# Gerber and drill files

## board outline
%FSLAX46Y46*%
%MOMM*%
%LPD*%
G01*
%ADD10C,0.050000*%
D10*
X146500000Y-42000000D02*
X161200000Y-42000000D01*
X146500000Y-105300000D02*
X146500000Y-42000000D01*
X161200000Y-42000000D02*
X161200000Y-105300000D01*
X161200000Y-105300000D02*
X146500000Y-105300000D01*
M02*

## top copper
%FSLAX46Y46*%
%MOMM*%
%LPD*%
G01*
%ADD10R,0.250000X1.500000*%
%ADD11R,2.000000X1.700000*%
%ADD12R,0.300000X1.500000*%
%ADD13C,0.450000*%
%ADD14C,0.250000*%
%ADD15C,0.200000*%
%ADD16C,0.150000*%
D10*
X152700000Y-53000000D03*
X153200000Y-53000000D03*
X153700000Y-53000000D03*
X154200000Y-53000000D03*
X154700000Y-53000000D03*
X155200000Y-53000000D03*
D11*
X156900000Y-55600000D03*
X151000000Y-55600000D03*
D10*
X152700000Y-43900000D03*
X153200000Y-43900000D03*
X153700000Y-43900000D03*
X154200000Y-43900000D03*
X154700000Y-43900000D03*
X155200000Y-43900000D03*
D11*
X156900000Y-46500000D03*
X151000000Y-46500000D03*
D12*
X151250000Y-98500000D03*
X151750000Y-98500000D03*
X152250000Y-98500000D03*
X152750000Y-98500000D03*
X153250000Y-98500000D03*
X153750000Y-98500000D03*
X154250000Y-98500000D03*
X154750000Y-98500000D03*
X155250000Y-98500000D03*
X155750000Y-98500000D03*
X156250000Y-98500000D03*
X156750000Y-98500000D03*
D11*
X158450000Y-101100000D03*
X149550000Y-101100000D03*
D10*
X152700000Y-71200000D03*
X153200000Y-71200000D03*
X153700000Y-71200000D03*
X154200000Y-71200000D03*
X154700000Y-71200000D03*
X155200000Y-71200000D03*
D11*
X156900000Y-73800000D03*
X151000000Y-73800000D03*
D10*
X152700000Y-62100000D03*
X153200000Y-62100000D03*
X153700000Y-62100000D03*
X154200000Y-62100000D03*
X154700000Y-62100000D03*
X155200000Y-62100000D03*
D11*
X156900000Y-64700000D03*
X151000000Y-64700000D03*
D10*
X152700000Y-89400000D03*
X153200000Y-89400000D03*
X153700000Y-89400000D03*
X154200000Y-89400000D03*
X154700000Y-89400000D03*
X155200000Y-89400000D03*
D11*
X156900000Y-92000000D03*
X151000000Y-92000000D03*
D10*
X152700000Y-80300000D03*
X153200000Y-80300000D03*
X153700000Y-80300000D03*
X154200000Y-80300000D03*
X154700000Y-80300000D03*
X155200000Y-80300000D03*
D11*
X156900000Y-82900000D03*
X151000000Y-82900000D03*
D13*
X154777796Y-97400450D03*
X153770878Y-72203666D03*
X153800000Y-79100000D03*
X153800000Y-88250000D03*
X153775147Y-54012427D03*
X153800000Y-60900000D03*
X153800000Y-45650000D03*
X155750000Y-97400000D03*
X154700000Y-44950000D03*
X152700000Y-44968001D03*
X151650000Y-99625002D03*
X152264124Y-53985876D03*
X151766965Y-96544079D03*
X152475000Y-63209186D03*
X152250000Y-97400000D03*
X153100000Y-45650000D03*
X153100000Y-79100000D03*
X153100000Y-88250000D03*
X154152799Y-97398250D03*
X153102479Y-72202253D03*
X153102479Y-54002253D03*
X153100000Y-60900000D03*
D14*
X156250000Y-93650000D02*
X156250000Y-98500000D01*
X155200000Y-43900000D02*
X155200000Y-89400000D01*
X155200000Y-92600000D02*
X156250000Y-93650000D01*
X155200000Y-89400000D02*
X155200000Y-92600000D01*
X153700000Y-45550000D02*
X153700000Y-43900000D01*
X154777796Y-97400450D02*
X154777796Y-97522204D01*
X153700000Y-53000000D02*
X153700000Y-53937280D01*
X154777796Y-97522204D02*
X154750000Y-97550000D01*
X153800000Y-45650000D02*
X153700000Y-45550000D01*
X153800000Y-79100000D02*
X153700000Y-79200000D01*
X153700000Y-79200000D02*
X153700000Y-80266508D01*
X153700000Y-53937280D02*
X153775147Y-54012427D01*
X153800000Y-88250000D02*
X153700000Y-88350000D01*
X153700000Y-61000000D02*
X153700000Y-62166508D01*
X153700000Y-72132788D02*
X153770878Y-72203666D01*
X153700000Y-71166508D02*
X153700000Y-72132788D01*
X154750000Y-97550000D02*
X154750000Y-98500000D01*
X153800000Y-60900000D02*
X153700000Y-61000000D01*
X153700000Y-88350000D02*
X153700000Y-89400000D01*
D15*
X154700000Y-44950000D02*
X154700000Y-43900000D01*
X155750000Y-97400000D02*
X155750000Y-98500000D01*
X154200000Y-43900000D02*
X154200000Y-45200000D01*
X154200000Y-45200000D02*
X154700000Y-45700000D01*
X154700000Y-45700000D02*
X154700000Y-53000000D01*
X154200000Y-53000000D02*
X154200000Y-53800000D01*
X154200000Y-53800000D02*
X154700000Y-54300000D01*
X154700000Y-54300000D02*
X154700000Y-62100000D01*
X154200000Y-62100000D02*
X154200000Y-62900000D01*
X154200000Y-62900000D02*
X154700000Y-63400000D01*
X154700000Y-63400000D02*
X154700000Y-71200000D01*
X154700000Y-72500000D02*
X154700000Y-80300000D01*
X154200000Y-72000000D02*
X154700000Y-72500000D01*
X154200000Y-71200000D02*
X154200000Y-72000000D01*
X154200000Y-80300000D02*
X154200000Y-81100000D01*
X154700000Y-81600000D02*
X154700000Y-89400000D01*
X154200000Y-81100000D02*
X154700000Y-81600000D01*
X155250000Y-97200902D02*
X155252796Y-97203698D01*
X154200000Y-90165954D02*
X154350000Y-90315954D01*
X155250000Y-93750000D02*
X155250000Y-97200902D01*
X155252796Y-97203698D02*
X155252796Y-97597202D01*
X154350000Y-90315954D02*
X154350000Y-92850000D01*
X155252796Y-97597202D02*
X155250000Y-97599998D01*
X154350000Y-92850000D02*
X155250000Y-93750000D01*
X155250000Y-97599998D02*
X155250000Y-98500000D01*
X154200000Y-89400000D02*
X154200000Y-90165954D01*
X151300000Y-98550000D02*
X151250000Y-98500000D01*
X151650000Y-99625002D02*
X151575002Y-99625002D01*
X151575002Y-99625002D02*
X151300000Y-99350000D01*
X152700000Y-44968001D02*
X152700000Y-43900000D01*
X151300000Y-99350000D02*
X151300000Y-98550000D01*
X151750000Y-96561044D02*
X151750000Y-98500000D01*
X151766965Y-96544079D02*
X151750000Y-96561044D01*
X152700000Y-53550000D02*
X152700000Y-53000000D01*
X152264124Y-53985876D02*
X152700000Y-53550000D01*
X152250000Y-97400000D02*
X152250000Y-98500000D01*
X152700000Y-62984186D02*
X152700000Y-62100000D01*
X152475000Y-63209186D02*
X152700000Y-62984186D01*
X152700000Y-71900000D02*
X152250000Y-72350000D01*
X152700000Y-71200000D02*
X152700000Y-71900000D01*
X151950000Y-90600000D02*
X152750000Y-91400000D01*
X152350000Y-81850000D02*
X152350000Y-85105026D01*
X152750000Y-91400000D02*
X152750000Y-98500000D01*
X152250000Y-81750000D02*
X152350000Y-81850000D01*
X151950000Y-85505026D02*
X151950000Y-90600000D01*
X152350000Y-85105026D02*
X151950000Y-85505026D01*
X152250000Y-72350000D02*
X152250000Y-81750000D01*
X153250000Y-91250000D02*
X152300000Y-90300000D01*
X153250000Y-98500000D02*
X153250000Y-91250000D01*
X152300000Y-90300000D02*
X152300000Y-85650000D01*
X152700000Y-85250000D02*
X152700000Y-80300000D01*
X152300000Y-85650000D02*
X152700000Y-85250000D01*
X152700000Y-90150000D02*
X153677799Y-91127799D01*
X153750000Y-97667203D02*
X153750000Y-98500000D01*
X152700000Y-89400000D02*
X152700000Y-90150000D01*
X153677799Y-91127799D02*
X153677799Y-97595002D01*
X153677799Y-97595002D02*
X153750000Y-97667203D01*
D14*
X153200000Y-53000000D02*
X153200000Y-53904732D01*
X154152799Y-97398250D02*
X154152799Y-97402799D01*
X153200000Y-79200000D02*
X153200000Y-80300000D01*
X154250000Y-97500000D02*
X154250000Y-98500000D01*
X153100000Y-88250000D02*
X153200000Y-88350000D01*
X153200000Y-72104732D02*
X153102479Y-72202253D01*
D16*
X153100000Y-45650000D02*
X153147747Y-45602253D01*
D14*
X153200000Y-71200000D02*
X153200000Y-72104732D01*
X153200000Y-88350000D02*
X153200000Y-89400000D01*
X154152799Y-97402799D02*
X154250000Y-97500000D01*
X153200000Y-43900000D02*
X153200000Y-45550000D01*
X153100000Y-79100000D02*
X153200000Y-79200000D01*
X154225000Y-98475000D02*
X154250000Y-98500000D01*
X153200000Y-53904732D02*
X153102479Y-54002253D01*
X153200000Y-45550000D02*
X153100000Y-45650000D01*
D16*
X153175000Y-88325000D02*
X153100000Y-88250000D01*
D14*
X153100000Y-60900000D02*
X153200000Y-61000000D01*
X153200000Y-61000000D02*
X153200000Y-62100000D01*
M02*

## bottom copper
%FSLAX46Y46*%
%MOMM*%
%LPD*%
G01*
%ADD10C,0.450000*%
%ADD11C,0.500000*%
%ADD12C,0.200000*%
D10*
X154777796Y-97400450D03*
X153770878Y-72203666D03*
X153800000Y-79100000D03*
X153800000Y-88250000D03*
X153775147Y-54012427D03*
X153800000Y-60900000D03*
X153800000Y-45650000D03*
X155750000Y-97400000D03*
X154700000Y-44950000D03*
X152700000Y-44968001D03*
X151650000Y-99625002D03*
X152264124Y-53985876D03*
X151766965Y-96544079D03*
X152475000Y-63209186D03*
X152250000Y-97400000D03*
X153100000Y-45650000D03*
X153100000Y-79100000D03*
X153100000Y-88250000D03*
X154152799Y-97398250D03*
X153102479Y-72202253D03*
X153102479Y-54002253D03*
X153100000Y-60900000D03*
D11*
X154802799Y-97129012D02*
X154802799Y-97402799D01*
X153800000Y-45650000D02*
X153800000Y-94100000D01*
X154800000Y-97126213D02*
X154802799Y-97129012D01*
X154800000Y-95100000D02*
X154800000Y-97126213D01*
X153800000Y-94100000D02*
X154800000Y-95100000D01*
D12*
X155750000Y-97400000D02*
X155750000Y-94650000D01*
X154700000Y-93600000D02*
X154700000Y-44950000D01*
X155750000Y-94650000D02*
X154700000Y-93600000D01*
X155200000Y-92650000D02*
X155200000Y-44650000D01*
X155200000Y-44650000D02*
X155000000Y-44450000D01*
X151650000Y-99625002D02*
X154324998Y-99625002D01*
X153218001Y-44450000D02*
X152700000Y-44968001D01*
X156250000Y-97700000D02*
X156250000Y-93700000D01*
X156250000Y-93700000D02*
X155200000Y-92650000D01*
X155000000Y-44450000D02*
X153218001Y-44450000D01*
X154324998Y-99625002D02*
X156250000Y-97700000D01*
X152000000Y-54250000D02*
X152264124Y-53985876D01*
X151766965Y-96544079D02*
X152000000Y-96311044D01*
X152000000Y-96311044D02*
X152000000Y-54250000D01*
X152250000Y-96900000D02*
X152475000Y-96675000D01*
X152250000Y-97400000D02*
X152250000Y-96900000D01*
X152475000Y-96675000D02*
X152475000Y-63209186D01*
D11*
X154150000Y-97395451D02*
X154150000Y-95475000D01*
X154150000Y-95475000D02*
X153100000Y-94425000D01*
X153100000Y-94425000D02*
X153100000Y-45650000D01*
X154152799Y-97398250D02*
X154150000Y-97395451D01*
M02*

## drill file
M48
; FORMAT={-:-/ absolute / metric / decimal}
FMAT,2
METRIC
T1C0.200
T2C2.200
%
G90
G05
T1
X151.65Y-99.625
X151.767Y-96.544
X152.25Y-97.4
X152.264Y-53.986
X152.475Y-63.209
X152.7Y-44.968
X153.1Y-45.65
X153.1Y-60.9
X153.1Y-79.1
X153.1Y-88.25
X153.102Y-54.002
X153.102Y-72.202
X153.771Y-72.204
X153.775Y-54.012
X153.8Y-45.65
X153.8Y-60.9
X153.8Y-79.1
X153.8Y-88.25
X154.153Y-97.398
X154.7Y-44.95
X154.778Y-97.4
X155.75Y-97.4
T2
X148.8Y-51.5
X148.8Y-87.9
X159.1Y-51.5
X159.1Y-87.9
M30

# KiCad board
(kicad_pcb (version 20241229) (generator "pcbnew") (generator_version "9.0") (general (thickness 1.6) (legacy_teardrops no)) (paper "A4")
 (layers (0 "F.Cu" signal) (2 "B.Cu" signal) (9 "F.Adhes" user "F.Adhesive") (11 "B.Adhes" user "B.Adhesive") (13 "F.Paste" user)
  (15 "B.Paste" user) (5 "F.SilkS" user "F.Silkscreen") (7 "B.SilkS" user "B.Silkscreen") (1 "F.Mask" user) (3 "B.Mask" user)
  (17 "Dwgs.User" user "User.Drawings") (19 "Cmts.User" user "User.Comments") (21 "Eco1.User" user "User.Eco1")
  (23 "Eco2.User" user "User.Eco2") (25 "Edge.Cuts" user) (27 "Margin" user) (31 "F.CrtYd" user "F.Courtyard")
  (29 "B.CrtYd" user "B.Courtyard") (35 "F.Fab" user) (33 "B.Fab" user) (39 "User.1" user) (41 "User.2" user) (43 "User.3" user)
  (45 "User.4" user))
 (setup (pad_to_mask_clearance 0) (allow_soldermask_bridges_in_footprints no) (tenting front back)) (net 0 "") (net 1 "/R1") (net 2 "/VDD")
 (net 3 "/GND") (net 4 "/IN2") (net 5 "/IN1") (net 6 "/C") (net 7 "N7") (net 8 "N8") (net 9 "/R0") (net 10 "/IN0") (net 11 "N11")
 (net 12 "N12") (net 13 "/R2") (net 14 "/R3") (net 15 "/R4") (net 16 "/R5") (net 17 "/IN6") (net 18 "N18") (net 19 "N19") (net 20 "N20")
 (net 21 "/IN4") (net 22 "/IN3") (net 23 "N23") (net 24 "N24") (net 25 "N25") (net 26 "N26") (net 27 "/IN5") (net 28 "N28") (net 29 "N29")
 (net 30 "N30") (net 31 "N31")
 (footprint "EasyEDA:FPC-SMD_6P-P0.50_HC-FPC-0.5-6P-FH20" (layer "F.Cu") (at 153.95 54.3)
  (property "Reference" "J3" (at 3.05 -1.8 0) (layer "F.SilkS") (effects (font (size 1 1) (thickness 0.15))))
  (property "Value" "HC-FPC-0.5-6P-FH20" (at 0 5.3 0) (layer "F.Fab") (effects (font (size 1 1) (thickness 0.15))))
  (pad "1" smd rect (at -1.25 -1.3) (size 0.25 1.5) (layers "F.Cu" "F.Mask" "F.Paste") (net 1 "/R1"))
  (pad "2" smd rect (at -0.75 -1.3) (size 0.25 1.5) (layers "F.Cu" "F.Mask" "F.Paste") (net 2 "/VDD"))
  (pad "3" smd rect (at -0.25 -1.3) (size 0.25 1.5) (layers "F.Cu" "F.Mask" "F.Paste") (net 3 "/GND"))
  (pad "4" smd rect (at 0.25 -1.3) (size 0.25 1.5) (layers "F.Cu" "F.Mask" "F.Paste") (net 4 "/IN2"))
  (pad "5" smd rect (at 0.75 -1.3) (size 0.25 1.5) (layers "F.Cu" "F.Mask" "F.Paste") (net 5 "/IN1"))
  (pad "6" smd rect (at 1.25 -1.3) (size 0.25 1.5) (layers "F.Cu" "F.Mask" "F.Paste") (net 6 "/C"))
  (pad "7" smd rect (at 2.95 1.3) (size 2 1.7) (layers "F.Cu" "F.Mask" "F.Paste") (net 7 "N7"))
  (pad "8" smd rect (at -2.95 1.3) (size 2 1.7) (layers "F.Cu" "F.Mask" "F.Paste") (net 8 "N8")))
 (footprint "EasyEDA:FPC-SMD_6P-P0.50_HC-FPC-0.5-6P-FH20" (layer "F.Cu") (at 153.95 45.2)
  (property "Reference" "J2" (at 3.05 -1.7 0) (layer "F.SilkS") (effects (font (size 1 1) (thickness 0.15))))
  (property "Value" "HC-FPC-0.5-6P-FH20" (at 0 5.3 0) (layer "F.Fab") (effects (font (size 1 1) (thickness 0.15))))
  (pad "1" smd rect (at -1.25 -1.3) (size 0.25 1.5) (layers "F.Cu" "F.Mask" "F.Paste") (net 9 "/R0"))
  (pad "2" smd rect (at -0.75 -1.3) (size 0.25 1.5) (layers "F.Cu" "F.Mask" "F.Paste") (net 2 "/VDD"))
  (pad "3" smd rect (at -0.25 -1.3) (size 0.25 1.5) (layers "F.Cu" "F.Mask" "F.Paste") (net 3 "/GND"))
  (pad "4" smd rect (at 0.25 -1.3) (size 0.25 1.5) (layers "F.Cu" "F.Mask" "F.Paste") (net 5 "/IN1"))
  (pad "5" smd rect (at 0.75 -1.3) (size 0.25 1.5) (layers "F.Cu" "F.Mask" "F.Paste") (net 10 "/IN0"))
  (pad "6" smd rect (at 1.25 -1.3) (size 0.25 1.5) (layers "F.Cu" "F.Mask" "F.Paste") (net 6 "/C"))
  (pad "7" smd rect (at 2.95 1.3) (size 2 1.7) (layers "F.Cu" "F.Mask" "F.Paste") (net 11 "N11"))
  (pad "8" smd rect (at -2.95 1.3) (size 2 1.7) (layers "F.Cu" "F.Mask" "F.Paste") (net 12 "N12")))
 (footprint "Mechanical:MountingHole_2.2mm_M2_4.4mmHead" (layer "F.Cu") (at 148.8 87.9)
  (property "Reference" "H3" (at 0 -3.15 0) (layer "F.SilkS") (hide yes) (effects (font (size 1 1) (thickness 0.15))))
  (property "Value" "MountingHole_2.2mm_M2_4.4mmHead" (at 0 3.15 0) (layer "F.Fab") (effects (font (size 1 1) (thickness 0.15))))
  (pad "" np_thru_hole circle (at 0 0) (size 2.2 2.2) (drill 2.2) (layers "*.Cu" "*.Mask")))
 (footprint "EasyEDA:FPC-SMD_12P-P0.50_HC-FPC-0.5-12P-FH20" (layer "F.Cu") (at 154 99.8)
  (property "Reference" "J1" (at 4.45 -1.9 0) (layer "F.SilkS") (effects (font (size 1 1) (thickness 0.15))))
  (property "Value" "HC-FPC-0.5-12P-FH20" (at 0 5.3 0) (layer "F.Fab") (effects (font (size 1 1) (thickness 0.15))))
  (pad "1" smd rect (at -2.75 -1.3) (size 0.3 1.5) (layers "F.Cu" "F.Mask" "F.Paste") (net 9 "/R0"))
  (pad "2" smd rect (at -2.25 -1.3) (size 0.3 1.5) (layers "F.Cu" "F.Mask" "F.Paste") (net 1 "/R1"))
  (pad "3" smd rect (at -1.75 -1.3) (size 0.3 1.5) (layers "F.Cu" "F.Mask" "F.Paste") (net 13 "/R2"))
  (pad "4" smd rect (at -1.25 -1.3) (size 0.3 1.5) (layers "F.Cu" "F.Mask" "F.Paste") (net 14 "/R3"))
  (pad "5" smd rect (at -0.75 -1.3) (size 0.3 1.5) (layers "F.Cu" "F.Mask" "F.Paste") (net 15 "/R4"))
  (pad "6" smd rect (at -0.25 -1.3) (size 0.3 1.5) (layers "F.Cu" "F.Mask" "F.Paste") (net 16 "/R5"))
  (pad "7" smd rect (at 0.25 -1.3) (size 0.3 1.5) (layers "F.Cu" "F.Mask" "F.Paste") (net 2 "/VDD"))
  (pad "8" smd rect (at 0.75 -1.3) (size 0.3 1.5) (layers "F.Cu" "F.Mask" "F.Paste") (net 3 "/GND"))
  (pad "9" smd rect (at 1.25 -1.3) (size 0.3 1.5) (layers "F.Cu" "F.Mask" "F.Paste") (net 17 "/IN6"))
  (pad "10" smd rect (at 1.75 -1.3) (size 0.3 1.5) (layers "F.Cu" "F.Mask" "F.Paste") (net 10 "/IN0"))
  (pad "11" smd rect (at 2.25 -1.3) (size 0.3 1.5) (layers "F.Cu" "F.Mask" "F.Paste") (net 6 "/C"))
  (pad "12" smd rect (at 2.75 -1.3) (size 0.3 1.5) (layers "F.Cu" "F.Mask" "F.Paste") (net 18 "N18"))
  (pad "13" smd rect (at 4.45 1.3) (size 2 1.7) (layers "F.Cu" "F.Mask" "F.Paste") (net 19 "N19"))
  (pad "14" smd rect (at -4.45 1.3) (size 2 1.7) (layers "F.Cu" "F.Mask" "F.Paste") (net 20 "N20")))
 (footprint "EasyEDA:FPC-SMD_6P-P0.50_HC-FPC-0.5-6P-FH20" (layer "F.Cu") (at 153.95 72.5)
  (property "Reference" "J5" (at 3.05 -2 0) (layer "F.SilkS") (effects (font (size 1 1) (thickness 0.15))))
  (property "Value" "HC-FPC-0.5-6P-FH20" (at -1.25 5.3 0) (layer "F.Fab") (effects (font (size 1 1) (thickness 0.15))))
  (pad "1" smd rect (at -1.25 -1.3) (size 0.25 1.5) (layers "F.Cu" "F.Mask" "F.Paste") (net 14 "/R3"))
  (pad "2" smd rect (at -0.75 -1.3) (size 0.25 1.5) (layers "F.Cu" "F.Mask" "F.Paste") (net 2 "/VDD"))
  (pad "3" smd rect (at -0.25 -1.3) (size 0.25 1.5) (layers "F.Cu" "F.Mask" "F.Paste") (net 3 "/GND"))
  (pad "4" smd rect (at 0.25 -1.3) (size 0.25 1.5) (layers "F.Cu" "F.Mask" "F.Paste") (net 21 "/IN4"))
  (pad "5" smd rect (at 0.75 -1.3) (size 0.25 1.5) (layers "F.Cu" "F.Mask" "F.Paste") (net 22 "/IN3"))
  (pad "6" smd rect (at 1.25 -1.3) (size 0.25 1.5) (layers "F.Cu" "F.Mask" "F.Paste") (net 6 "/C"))
  (pad "7" smd rect (at 2.95 1.3) (size 2 1.7) (layers "F.Cu" "F.Mask" "F.Paste") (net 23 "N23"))
  (pad "8" smd rect (at -2.95 1.3) (size 2 1.7) (layers "F.Cu" "F.Mask" "F.Paste") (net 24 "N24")))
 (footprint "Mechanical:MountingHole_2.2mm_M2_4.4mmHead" (layer "F.Cu") (at 159.1 51.5)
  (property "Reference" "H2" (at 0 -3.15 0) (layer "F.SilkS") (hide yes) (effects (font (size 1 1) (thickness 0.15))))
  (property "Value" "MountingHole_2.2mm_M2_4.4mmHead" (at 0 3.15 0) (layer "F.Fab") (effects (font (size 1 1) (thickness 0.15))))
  (pad "" np_thru_hole circle (at 0 0) (size 2.2 2.2) (drill 2.2) (layers "*.Cu" "*.Mask")))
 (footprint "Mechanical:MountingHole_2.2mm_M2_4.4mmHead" (layer "F.Cu") (at 148.8 51.5)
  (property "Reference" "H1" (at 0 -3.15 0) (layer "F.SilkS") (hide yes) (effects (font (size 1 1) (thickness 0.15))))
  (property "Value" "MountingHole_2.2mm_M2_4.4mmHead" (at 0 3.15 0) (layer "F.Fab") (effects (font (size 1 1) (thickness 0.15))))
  (pad "" np_thru_hole circle (at 0 0) (size 2.2 2.2) (drill 2.2) (layers "*.Cu" "*.Mask")))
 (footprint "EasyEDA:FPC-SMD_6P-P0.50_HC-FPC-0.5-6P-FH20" (layer "F.Cu") (at 153.95 63.4)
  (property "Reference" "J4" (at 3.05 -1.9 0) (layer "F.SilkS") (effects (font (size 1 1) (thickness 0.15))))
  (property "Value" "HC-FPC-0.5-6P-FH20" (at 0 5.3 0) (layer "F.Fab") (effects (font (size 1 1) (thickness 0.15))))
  (pad "1" smd rect (at -1.25 -1.3) (size 0.25 1.5) (layers "F.Cu" "F.Mask" "F.Paste") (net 13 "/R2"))
  (pad "2" smd rect (at -0.75 -1.3) (size 0.25 1.5) (layers "F.Cu" "F.Mask" "F.Paste") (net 2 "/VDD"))
  (pad "3" smd rect (at -0.25 -1.3) (size 0.25 1.5) (layers "F.Cu" "F.Mask" "F.Paste") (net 3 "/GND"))
  (pad "4" smd rect (at 0.25 -1.3) (size 0.25 1.5) (layers "F.Cu" "F.Mask" "F.Paste") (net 22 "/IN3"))
  (pad "5" smd rect (at 0.75 -1.3) (size 0.25 1.5) (layers "F.Cu" "F.Mask" "F.Paste") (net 4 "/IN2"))
  (pad "6" smd rect (at 1.25 -1.3) (size 0.25 1.5) (layers "F.Cu" "F.Mask" "F.Paste") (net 6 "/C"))
  (pad "7" smd rect (at 2.95 1.3) (size 2 1.7) (layers "F.Cu" "F.Mask" "F.Paste") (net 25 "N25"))
  (pad "8" smd rect (at -2.95 1.3) (size 2 1.7) (layers "F.Cu" "F.Mask" "F.Paste") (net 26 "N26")))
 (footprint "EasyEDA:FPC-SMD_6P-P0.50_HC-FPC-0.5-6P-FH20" (layer "F.Cu") (at 153.95 90.7)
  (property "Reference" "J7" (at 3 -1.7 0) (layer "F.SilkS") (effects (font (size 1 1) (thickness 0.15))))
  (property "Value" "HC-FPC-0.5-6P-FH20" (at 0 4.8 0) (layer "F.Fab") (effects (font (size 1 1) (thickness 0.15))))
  (pad "1" smd rect (at -1.25 -1.3) (size 0.25 1.5) (layers "F.Cu" "F.Mask" "F.Paste") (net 16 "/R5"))
  (pad "2" smd rect (at -0.75 -1.3) (size 0.25 1.5) (layers "F.Cu" "F.Mask" "F.Paste") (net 2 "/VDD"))
  (pad "3" smd rect (at -0.25 -1.3) (size 0.25 1.5) (layers "F.Cu" "F.Mask" "F.Paste") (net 3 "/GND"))
  (pad "4" smd rect (at 0.25 -1.3) (size 0.25 1.5) (layers "F.Cu" "F.Mask" "F.Paste") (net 17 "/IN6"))
  (pad "5" smd rect (at 0.75 -1.3) (size 0.25 1.5) (layers "F.Cu" "F.Mask" "F.Paste") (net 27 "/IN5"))
  (pad "6" smd rect (at 1.25 -1.3) (size 0.25 1.5) (layers "F.Cu" "F.Mask" "F.Paste") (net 6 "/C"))
  (pad "7" smd rect (at 2.95 1.3) (size 2 1.7) (layers "F.Cu" "F.Mask" "F.Paste") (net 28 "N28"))
  (pad "8" smd rect (at -2.95 1.3) (size 2 1.7) (layers "F.Cu" "F.Mask" "F.Paste") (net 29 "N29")))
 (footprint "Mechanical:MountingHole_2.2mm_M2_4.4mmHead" (layer "F.Cu") (at 159.1 87.9)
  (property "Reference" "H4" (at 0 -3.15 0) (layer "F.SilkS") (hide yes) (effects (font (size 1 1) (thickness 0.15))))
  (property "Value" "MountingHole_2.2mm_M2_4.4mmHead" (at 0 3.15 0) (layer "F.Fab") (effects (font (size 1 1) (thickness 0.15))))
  (pad "" np_thru_hole circle (at 0 0) (size 2.2 2.2) (drill 2.2) (layers "*.Cu" "*.Mask")))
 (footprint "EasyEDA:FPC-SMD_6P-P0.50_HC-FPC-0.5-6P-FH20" (layer "F.Cu") (at 153.95 81.6)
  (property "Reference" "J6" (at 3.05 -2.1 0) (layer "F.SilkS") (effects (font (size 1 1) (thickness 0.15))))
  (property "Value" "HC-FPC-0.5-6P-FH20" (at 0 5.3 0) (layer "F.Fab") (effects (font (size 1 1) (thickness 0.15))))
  (pad "1" smd rect (at -1.25 -1.3) (size 0.25 1.5) (layers "F.Cu" "F.Mask" "F.Paste") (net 15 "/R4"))
  (pad "2" smd rect (at -0.75 -1.3) (size 0.25 1.5) (layers "F.Cu" "F.Mask" "F.Paste") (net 2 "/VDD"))
  (pad "3" smd rect (at -0.25 -1.3) (size 0.25 1.5) (layers "F.Cu" "F.Mask" "F.Paste") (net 3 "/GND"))
  (pad "4" smd rect (at 0.25 -1.3) (size 0.25 1.5) (layers "F.Cu" "F.Mask" "F.Paste") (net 27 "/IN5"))
  (pad "5" smd rect (at 0.75 -1.3) (size 0.25 1.5) (layers "F.Cu" "F.Mask" "F.Paste") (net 21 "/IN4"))
  (pad "6" smd rect (at 1.25 -1.3) (size 0.25 1.5) (layers "F.Cu" "F.Mask" "F.Paste") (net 6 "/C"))
  (pad "7" smd rect (at 2.95 1.3) (size 2 1.7) (layers "F.Cu" "F.Mask" "F.Paste") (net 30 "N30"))
  (pad "8" smd rect (at -2.95 1.3) (size 2 1.7) (layers "F.Cu" "F.Mask" "F.Paste") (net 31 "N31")))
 (gr_line (start 146.5 42) (end 161.2 42) (stroke (width 0.05) (type default)) (layer "Edge.Cuts"))
 (gr_line (start 146.5 105.3) (end 146.5 42) (stroke (width 0.05) (type default)) (layer "Edge.Cuts"))
 (gr_line (start 161.2 42) (end 161.2 105.3) (stroke (width 0.05) (type default)) (layer "Edge.Cuts"))
 (gr_line (start 161.2 105.3) (end 146.5 105.3) (stroke (width 0.05) (type default)) (layer "Edge.Cuts"))
 (segment (start 156.25 93.65) (end 156.25 98.5) (width 0.25) (layer "F.Cu") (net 6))
 (segment (start 155.2 43.9) (end 155.2 89.4) (width 0.25) (layer "F.Cu") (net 6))
 (segment (start 155.2 92.6) (end 156.25 93.65) (width 0.25) (layer "F.Cu") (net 6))
 (segment (start 155.2 89.4) (end 155.2 92.6) (width 0.25) (layer "F.Cu") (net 6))
 (segment (start 153.7 45.55) (end 153.7 43.9) (width 0.25) (layer "F.Cu") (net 3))
 (segment (start 154.777796 97.40045) (end 154.777796 97.522204) (width 0.25) (layer "F.Cu") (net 3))
 (segment (start 153.7 53) (end 153.7 53.93728) (width 0.25) (layer "F.Cu") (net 3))
 (segment (start 154.777796 97.522204) (end 154.75 97.55) (width 0.25) (layer "F.Cu") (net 3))
 (segment (start 153.8 45.65) (end 153.7 45.55) (width 0.25) (layer "F.Cu") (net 3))
 (segment (start 153.8 79.1) (end 153.7 79.2) (width 0.25) (layer "F.Cu") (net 3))
 (segment (start 153.7 79.2) (end 153.7 80.266508) (width 0.25) (layer "F.Cu") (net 3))
 (segment (start 153.7 53.93728) (end 153.775147 54.012427) (width 0.25) (layer "F.Cu") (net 3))
 (segment (start 153.8 88.25) (end 153.7 88.35) (width 0.25) (layer "F.Cu") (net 3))
 (segment (start 153.7 61) (end 153.7 62.166508) (width 0.25) (layer "F.Cu") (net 3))
 (segment (start 153.7 72.132788) (end 153.770878 72.203666) (width 0.25) (layer "F.Cu") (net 3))
 (segment (start 153.7 71.166508) (end 153.7 72.132788) (width 0.25) (layer "F.Cu") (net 3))
 (segment (start 154.75 97.55) (end 154.75 98.5) (width 0.25) (layer "F.Cu") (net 3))
 (segment (start 153.8 60.9) (end 153.7 61) (width 0.25) (layer "F.Cu") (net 3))
 (segment (start 153.7 88.35) (end 153.7 89.4) (width 0.25) (layer "F.Cu") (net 3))
 (via (at 154.777796 97.40045) (size 0.45) (drill 0.2) (layers "F.Cu" "B.Cu") (free yes) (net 3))
 (via (at 153.770878 72.203666) (size 0.45) (drill 0.2) (layers "F.Cu" "B.Cu") (free yes) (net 3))
 (via (at 153.8 79.1) (size 0.45) (drill 0.2) (layers "F.Cu" "B.Cu") (free yes) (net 3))
 (via (at 153.8 88.25) (size 0.45) (drill 0.2) (layers "F.Cu" "B.Cu") (free yes) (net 3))
 (via (at 153.775147 54.012427) (size 0.45) (drill 0.2) (layers "F.Cu" "B.Cu") (free yes) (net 3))
 (via (at 153.8 60.9) (size 0.45) (drill 0.2) (layers "F.Cu" "B.Cu") (free yes) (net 3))
 (via (at 153.8 45.65) (size 0.45) (drill 0.2) (layers "F.Cu" "B.Cu") (free yes) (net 3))
 (segment (start 154.802799 97.129012) (end 154.802799 97.402799) (width 0.5) (layer "B.Cu") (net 3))
 (segment (start 153.8 45.65) (end 153.8 94.1) (width 0.5) (layer "B.Cu") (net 3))
 (segment (start 154.8 97.126213) (end 154.802799 97.129012) (width 0.5) (layer "B.Cu") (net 3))
 (segment (start 154.8 95.1) (end 154.8 97.126213) (width 0.5) (layer "B.Cu") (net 3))
 (segment (start 153.8 94.1) (end 154.8 95.1) (width 0.5) (layer "B.Cu") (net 3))
 (segment (start 154.7 44.95) (end 154.7 43.9) (width 0.2) (layer "F.Cu") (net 10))
 (segment (start 155.75 97.4) (end 155.75 98.5) (width 0.2) (layer "F.Cu") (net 10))
 (via (at 155.75 97.4) (size 0.45) (drill 0.2) (layers "F.Cu" "B.Cu") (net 10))
 (via (at 154.7 44.95) (size 0.45) (drill 0.2) (layers "F.Cu" "B.Cu") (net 10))
 (segment (start 155.75 97.4) (end 155.75 94.65) (width 0.2) (layer "B.Cu") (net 10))
 (segment (start 154.7 93.6) (end 154.7 44.95) (width 0.2) (layer "B.Cu") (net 10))
 (segment (start 155.75 94.65) (end 154.7 93.6) (width 0.2) (layer "B.Cu") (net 10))
 (segment (start 154.2 43.9) (end 154.2 45.2) (width 0.2) (layer "F.Cu") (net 5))
 (segment (start 154.2 45.2) (end 154.7 45.7) (width 0.2) (layer "F.Cu") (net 5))
 (segment (start 154.7 45.7) (end 154.7 53) (width 0.2) (layer "F.Cu") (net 5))
 (segment (start 154.2 53) (end 154.2 53.8) (width 0.2) (layer "F.Cu") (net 4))
 (segment (start 154.2 53.8) (end 154.7 54.3) (width 0.2) (layer "F.Cu") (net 4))
 (segment (start 154.7 54.3) (end 154.7 62.1) (width 0.2) (layer "F.Cu") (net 4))
 (segment (start 154.2 62.1) (end 154.2 62.9) (width 0.2) (layer "F.Cu") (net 22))
 (segment (start 154.2 62.9) (end 154.7 63.4) (width 0.2) (layer "F.Cu") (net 22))
 (segment (start 154.7 63.4) (end 154.7 71.2) (width 0.2) (layer "F.Cu") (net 22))
 (segment (start 154.7 72.5) (end 154.7 80.3) (width 0.2) (layer "F.Cu") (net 21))
 (segment (start 154.2 72) (end 154.7 72.5) (width 0.2) (layer "F.Cu") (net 21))
 (segment (start 154.2 71.2) (end 154.2 72) (width 0.2) (layer "F.Cu") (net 21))
 (segment (start 154.2 80.3) (end 154.2 81.1) (width 0.2) (layer "F.Cu") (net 27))
 (segment (start 154.7 81.6) (end 154.7 89.4) (width 0.2) (layer "F.Cu") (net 27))
 (segment (start 154.2 81.1) (end 154.7 81.6) (width 0.2) (layer "F.Cu") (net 27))
 (segment (start 155.25 97.200902) (end 155.252796 97.203698) (width 0.2) (layer "F.Cu") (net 17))
 (segment (start 154.2 90.165954) (end 154.35 90.315954) (width 0.2) (layer "F.Cu") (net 17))
 (segment (start 155.25 93.75) (end 155.25 97.200902) (width 0.2) (layer "F.Cu") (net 17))
 (segment (start 155.252796 97.203698) (end 155.252796 97.597202) (width 0.2) (layer "F.Cu") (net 17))
 (segment (start 154.35 90.315954) (end 154.35 92.85) (width 0.2) (layer "F.Cu") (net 17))
 (segment (start 155.252796 97.597202) (end 155.25 97.599998) (width 0.2) (layer "F.Cu") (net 17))
 (segment (start 154.35 92.85) (end 155.25 93.75) (width 0.2) (layer "F.Cu") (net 17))
 (segment (start 155.25 97.599998) (end 155.25 98.5) (width 0.2) (layer "F.Cu") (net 17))
 (segment (start 154.2 89.4) (end 154.2 90.165954) (width 0.2) (layer "F.Cu") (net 17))
 (segment (start 151.3 98.55) (end 151.25 98.5) (width 0.2) (layer "F.Cu") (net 9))
 (segment (start 151.65 99.625002) (end 151.575002 99.625002) (width 0.2) (layer "F.Cu") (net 9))
 (segment (start 151.575002 99.625002) (end 151.3 99.35) (width 0.2) (layer "F.Cu") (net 9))
 (segment (start 152.7 44.968001) (end 152.7 43.9) (width 0.2) (layer "F.Cu") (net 9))
 (segment (start 151.3 99.35) (end 151.3 98.55) (width 0.2) (layer "F.Cu") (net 9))
 (via (at 152.7 44.968001) (size 0.45) (drill 0.2) (layers "F.Cu" "B.Cu") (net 9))
 (via (at 151.65 99.625002) (size 0.45) (drill 0.2) (layers "F.Cu" "B.Cu") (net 9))
 (segment (start 155.2 92.65) (end 155.2 44.65) (width 0.2) (layer "B.Cu") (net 9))
 (segment (start 155.2 44.65) (end 155 44.45) (width 0.2) (layer "B.Cu") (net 9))
 (segment (start 151.65 99.625002) (end 154.324998 99.625002) (width 0.2) (layer "B.Cu") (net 9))
 (segment (start 153.218001 44.45) (end 152.7 44.968001) (width 0.2) (layer "B.Cu") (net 9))
 (segment (start 156.25 97.7) (end 156.25 93.7) (width 0.2) (layer "B.Cu") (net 9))
 (segment (start 156.25 93.7) (end 155.2 92.65) (width 0.2) (layer "B.Cu") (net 9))
 (segment (start 155 44.45) (end 153.218001 44.45) (width 0.2) (layer "B.Cu") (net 9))
 (segment (start 154.324998 99.625002) (end 156.25 97.7) (width 0.2) (layer "B.Cu") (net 9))
 (segment (start 151.75 96.561044) (end 151.75 98.5) (width 0.2) (layer "F.Cu") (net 1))
 (segment (start 151.766965 96.544079) (end 151.75 96.561044) (width 0.2) (layer "F.Cu") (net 1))
 (segment (start 152.7 53.55) (end 152.7 53) (width 0.2) (layer "F.Cu") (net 1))
 (segment (start 152.264124 53.985876) (end 152.7 53.55) (width 0.2) (layer "F.Cu") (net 1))
 (via (at 152.264124 53.985876) (size 0.45) (drill 0.2) (layers "F.Cu" "B.Cu") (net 1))
 (via (at 151.766965 96.544079) (size 0.45) (drill 0.2) (layers "F.Cu" "B.Cu") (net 1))
 (segment (start 152 54.25) (end 152.264124 53.985876) (width 0.2) (layer "B.Cu") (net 1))
 (segment (start 151.766965 96.544079) (end 152 96.311044) (width 0.2) (layer "B.Cu") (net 1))
 (segment (start 152 96.311044) (end 152 54.25) (width 0.2) (layer "B.Cu") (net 1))
 (segment (start 152.25 97.4) (end 152.25 98.5) (width 0.2) (layer "F.Cu") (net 13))
 (segment (start 152.7 62.984186) (end 152.7 62.1) (width 0.2) (layer "F.Cu") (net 13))
 (segment (start 152.475 63.209186) (end 152.7 62.984186) (width 0.2) (layer "F.Cu") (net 13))
 (via (at 152.475 63.209186) (size 0.45) (drill 0.2) (layers "F.Cu" "B.Cu") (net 13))
 (via (at 152.25 97.4) (size 0.45) (drill 0.2) (layers "F.Cu" "B.Cu") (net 13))
 (segment (start 152.25 96.9) (end 152.475 96.675) (width 0.2) (layer "B.Cu") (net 13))
 (segment (start 152.25 97.4) (end 152.25 96.9) (width 0.2) (layer "B.Cu") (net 13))
 (segment (start 152.475 96.675) (end 152.475 63.209186) (width 0.2) (layer "B.Cu") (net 13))
 (segment (start 152.7 71.9) (end 152.25 72.35) (width 0.2) (layer "F.Cu") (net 14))
 (segment (start 152.7 71.2) (end 152.7 71.9) (width 0.2) (layer "F.Cu") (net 14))
 (segment (start 151.95 90.6) (end 152.75 91.4) (width 0.2) (layer "F.Cu") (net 14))
 (segment (start 152.35 81.85) (end 152.35 85.105026) (width 0.2) (layer "F.Cu") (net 14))
 (segment (start 152.75 91.4) (end 152.75 98.5) (width 0.2) (layer "F.Cu") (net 14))
 (segment (start 152.25 81.75) (end 152.35 81.85) (width 0.2) (layer "F.Cu") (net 14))
 (segment (start 151.95 85.505026) (end 151.95 90.6) (width 0.2) (layer "F.Cu") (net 14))
 (segment (start 152.35 85.105026) (end 151.95 85.505026) (width 0.2) (layer "F.Cu") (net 14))
 (segment (start 152.25 72.35) (end 152.25 81.75) (width 0.2) (layer "F.Cu") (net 14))
 (segment (start 153.25 91.25) (end 152.3 90.3) (width 0.2) (layer "F.Cu") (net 15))
 (segment (start 153.25 98.5) (end 153.25 91.25) (width 0.2) (layer "F.Cu") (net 15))
 (segment (start 152.3 90.3) (end 152.3 85.65) (width 0.2) (layer "F.Cu") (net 15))
 (segment (start 152.7 85.25) (end 152.7 80.3) (width 0.2) (layer "F.Cu") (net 15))
 (segment (start 152.3 85.65) (end 152.7 85.25) (width 0.2) (layer "F.Cu") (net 15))
 (segment (start 152.7 90.15) (end 153.677799 91.127799) (width 0.2) (layer "F.Cu") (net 16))
 (segment (start 153.75 97.667203) (end 153.75 98.5) (width 0.2) (layer "F.Cu") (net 16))
 (segment (start 152.7 89.4) (end 152.7 90.15) (width 0.2) (layer "F.Cu") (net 16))
 (segment (start 153.677799 91.127799) (end 153.677799 97.595002) (width 0.2) (layer "F.Cu") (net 16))
 (segment (start 153.677799 97.595002) (end 153.75 97.667203) (width 0.2) (layer "F.Cu") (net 16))
 (segment (start 153.2 53) (end 153.2 53.904732) (width 0.25) (layer "F.Cu") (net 2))
 (segment (start 154.152799 97.39825) (end 154.152799 97.402799) (width 0.25) (layer "F.Cu") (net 2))
 (segment (start 153.2 79.2) (end 153.2 80.3) (width 0.25) (layer "F.Cu") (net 2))
 (segment (start 154.25 97.5) (end 154.25 98.5) (width 0.25) (layer "F.Cu") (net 2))
 (segment (start 153.1 88.25) (end 153.2 88.35) (width 0.25) (layer "F.Cu") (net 2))
 (segment (start 153.2 72.104732) (end 153.102479 72.202253) (width 0.25) (layer "F.Cu") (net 2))
 (segment (start 153.1 45.65) (end 153.147747 45.602253) (width 0.15) (layer "F.Cu") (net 2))
 (segment (start 153.2 71.2) (end 153.2 72.104732) (width 0.25) (layer "F.Cu") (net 2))
 (segment (start 153.2 88.35) (end 153.2 89.4) (width 0.25) (layer "F.Cu") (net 2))
 (segment (start 154.152799 97.402799) (end 154.25 97.5) (width 0.25) (layer "F.Cu") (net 2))
 (segment (start 153.2 43.9) (end 153.2 45.55) (width 0.25) (layer "F.Cu") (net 2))
 (segment (start 153.1 79.1) (end 153.2 79.2) (width 0.25) (layer "F.Cu") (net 2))
 (segment (start 154.225 98.475) (end 154.25 98.5) (width 0.25) (layer "F.Cu") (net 2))
 (segment (start 153.2 53.904732) (end 153.102479 54.002253) (width 0.25) (layer "F.Cu") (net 2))
 (segment (start 153.2 45.55) (end 153.1 45.65) (width 0.25) (layer "F.Cu") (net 2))
 (segment (start 153.175 88.325) (end 153.1 88.25) (width 0.15) (layer "F.Cu") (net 2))
 (segment (start 153.1 60.9) (end 153.2 61) (width 0.25) (layer "F.Cu") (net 2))
 (segment (start 153.2 61) (end 153.2 62.1) (width 0.25) (layer "F.Cu") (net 2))
 (via (at 153.1 45.65) (size 0.45) (drill 0.2) (layers "F.Cu" "B.Cu") (free yes) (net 2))
 (via (at 153.1 79.1) (size 0.45) (drill 0.2) (layers "F.Cu" "B.Cu") (free yes) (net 2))
 (via (at 153.1 88.25) (size 0.45) (drill 0.2) (layers "F.Cu" "B.Cu") (free yes) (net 2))
 (via (at 154.152799 97.39825) (size 0.45) (drill 0.2) (layers "F.Cu" "B.Cu") (free yes) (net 2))
 (via (at 153.102479 72.202253) (size 0.45) (drill 0.2) (layers "F.Cu" "B.Cu") (free yes) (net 2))
 (via (at 153.102479 54.002253) (size 0.45) (drill 0.2) (layers "F.Cu" "B.Cu") (free yes) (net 2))
 (via (at 153.1 60.9) (size 0.45) (drill 0.2) (layers "F.Cu" "B.Cu") (free yes) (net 2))
 (segment (start 154.15 97.395451) (end 154.15 95.475) (width 0.5) (layer "B.Cu") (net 2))
 (segment (start 154.15 95.475) (end 153.1 94.425) (width 0.5) (layer "B.Cu") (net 2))
 (segment (start 153.1 94.425) (end 153.1 45.65) (width 0.5) (layer "B.Cu") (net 2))
 (segment (start 154.152799 97.39825) (end 154.15 97.395451) (width 0.5) (layer "B.Cu") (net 2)))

